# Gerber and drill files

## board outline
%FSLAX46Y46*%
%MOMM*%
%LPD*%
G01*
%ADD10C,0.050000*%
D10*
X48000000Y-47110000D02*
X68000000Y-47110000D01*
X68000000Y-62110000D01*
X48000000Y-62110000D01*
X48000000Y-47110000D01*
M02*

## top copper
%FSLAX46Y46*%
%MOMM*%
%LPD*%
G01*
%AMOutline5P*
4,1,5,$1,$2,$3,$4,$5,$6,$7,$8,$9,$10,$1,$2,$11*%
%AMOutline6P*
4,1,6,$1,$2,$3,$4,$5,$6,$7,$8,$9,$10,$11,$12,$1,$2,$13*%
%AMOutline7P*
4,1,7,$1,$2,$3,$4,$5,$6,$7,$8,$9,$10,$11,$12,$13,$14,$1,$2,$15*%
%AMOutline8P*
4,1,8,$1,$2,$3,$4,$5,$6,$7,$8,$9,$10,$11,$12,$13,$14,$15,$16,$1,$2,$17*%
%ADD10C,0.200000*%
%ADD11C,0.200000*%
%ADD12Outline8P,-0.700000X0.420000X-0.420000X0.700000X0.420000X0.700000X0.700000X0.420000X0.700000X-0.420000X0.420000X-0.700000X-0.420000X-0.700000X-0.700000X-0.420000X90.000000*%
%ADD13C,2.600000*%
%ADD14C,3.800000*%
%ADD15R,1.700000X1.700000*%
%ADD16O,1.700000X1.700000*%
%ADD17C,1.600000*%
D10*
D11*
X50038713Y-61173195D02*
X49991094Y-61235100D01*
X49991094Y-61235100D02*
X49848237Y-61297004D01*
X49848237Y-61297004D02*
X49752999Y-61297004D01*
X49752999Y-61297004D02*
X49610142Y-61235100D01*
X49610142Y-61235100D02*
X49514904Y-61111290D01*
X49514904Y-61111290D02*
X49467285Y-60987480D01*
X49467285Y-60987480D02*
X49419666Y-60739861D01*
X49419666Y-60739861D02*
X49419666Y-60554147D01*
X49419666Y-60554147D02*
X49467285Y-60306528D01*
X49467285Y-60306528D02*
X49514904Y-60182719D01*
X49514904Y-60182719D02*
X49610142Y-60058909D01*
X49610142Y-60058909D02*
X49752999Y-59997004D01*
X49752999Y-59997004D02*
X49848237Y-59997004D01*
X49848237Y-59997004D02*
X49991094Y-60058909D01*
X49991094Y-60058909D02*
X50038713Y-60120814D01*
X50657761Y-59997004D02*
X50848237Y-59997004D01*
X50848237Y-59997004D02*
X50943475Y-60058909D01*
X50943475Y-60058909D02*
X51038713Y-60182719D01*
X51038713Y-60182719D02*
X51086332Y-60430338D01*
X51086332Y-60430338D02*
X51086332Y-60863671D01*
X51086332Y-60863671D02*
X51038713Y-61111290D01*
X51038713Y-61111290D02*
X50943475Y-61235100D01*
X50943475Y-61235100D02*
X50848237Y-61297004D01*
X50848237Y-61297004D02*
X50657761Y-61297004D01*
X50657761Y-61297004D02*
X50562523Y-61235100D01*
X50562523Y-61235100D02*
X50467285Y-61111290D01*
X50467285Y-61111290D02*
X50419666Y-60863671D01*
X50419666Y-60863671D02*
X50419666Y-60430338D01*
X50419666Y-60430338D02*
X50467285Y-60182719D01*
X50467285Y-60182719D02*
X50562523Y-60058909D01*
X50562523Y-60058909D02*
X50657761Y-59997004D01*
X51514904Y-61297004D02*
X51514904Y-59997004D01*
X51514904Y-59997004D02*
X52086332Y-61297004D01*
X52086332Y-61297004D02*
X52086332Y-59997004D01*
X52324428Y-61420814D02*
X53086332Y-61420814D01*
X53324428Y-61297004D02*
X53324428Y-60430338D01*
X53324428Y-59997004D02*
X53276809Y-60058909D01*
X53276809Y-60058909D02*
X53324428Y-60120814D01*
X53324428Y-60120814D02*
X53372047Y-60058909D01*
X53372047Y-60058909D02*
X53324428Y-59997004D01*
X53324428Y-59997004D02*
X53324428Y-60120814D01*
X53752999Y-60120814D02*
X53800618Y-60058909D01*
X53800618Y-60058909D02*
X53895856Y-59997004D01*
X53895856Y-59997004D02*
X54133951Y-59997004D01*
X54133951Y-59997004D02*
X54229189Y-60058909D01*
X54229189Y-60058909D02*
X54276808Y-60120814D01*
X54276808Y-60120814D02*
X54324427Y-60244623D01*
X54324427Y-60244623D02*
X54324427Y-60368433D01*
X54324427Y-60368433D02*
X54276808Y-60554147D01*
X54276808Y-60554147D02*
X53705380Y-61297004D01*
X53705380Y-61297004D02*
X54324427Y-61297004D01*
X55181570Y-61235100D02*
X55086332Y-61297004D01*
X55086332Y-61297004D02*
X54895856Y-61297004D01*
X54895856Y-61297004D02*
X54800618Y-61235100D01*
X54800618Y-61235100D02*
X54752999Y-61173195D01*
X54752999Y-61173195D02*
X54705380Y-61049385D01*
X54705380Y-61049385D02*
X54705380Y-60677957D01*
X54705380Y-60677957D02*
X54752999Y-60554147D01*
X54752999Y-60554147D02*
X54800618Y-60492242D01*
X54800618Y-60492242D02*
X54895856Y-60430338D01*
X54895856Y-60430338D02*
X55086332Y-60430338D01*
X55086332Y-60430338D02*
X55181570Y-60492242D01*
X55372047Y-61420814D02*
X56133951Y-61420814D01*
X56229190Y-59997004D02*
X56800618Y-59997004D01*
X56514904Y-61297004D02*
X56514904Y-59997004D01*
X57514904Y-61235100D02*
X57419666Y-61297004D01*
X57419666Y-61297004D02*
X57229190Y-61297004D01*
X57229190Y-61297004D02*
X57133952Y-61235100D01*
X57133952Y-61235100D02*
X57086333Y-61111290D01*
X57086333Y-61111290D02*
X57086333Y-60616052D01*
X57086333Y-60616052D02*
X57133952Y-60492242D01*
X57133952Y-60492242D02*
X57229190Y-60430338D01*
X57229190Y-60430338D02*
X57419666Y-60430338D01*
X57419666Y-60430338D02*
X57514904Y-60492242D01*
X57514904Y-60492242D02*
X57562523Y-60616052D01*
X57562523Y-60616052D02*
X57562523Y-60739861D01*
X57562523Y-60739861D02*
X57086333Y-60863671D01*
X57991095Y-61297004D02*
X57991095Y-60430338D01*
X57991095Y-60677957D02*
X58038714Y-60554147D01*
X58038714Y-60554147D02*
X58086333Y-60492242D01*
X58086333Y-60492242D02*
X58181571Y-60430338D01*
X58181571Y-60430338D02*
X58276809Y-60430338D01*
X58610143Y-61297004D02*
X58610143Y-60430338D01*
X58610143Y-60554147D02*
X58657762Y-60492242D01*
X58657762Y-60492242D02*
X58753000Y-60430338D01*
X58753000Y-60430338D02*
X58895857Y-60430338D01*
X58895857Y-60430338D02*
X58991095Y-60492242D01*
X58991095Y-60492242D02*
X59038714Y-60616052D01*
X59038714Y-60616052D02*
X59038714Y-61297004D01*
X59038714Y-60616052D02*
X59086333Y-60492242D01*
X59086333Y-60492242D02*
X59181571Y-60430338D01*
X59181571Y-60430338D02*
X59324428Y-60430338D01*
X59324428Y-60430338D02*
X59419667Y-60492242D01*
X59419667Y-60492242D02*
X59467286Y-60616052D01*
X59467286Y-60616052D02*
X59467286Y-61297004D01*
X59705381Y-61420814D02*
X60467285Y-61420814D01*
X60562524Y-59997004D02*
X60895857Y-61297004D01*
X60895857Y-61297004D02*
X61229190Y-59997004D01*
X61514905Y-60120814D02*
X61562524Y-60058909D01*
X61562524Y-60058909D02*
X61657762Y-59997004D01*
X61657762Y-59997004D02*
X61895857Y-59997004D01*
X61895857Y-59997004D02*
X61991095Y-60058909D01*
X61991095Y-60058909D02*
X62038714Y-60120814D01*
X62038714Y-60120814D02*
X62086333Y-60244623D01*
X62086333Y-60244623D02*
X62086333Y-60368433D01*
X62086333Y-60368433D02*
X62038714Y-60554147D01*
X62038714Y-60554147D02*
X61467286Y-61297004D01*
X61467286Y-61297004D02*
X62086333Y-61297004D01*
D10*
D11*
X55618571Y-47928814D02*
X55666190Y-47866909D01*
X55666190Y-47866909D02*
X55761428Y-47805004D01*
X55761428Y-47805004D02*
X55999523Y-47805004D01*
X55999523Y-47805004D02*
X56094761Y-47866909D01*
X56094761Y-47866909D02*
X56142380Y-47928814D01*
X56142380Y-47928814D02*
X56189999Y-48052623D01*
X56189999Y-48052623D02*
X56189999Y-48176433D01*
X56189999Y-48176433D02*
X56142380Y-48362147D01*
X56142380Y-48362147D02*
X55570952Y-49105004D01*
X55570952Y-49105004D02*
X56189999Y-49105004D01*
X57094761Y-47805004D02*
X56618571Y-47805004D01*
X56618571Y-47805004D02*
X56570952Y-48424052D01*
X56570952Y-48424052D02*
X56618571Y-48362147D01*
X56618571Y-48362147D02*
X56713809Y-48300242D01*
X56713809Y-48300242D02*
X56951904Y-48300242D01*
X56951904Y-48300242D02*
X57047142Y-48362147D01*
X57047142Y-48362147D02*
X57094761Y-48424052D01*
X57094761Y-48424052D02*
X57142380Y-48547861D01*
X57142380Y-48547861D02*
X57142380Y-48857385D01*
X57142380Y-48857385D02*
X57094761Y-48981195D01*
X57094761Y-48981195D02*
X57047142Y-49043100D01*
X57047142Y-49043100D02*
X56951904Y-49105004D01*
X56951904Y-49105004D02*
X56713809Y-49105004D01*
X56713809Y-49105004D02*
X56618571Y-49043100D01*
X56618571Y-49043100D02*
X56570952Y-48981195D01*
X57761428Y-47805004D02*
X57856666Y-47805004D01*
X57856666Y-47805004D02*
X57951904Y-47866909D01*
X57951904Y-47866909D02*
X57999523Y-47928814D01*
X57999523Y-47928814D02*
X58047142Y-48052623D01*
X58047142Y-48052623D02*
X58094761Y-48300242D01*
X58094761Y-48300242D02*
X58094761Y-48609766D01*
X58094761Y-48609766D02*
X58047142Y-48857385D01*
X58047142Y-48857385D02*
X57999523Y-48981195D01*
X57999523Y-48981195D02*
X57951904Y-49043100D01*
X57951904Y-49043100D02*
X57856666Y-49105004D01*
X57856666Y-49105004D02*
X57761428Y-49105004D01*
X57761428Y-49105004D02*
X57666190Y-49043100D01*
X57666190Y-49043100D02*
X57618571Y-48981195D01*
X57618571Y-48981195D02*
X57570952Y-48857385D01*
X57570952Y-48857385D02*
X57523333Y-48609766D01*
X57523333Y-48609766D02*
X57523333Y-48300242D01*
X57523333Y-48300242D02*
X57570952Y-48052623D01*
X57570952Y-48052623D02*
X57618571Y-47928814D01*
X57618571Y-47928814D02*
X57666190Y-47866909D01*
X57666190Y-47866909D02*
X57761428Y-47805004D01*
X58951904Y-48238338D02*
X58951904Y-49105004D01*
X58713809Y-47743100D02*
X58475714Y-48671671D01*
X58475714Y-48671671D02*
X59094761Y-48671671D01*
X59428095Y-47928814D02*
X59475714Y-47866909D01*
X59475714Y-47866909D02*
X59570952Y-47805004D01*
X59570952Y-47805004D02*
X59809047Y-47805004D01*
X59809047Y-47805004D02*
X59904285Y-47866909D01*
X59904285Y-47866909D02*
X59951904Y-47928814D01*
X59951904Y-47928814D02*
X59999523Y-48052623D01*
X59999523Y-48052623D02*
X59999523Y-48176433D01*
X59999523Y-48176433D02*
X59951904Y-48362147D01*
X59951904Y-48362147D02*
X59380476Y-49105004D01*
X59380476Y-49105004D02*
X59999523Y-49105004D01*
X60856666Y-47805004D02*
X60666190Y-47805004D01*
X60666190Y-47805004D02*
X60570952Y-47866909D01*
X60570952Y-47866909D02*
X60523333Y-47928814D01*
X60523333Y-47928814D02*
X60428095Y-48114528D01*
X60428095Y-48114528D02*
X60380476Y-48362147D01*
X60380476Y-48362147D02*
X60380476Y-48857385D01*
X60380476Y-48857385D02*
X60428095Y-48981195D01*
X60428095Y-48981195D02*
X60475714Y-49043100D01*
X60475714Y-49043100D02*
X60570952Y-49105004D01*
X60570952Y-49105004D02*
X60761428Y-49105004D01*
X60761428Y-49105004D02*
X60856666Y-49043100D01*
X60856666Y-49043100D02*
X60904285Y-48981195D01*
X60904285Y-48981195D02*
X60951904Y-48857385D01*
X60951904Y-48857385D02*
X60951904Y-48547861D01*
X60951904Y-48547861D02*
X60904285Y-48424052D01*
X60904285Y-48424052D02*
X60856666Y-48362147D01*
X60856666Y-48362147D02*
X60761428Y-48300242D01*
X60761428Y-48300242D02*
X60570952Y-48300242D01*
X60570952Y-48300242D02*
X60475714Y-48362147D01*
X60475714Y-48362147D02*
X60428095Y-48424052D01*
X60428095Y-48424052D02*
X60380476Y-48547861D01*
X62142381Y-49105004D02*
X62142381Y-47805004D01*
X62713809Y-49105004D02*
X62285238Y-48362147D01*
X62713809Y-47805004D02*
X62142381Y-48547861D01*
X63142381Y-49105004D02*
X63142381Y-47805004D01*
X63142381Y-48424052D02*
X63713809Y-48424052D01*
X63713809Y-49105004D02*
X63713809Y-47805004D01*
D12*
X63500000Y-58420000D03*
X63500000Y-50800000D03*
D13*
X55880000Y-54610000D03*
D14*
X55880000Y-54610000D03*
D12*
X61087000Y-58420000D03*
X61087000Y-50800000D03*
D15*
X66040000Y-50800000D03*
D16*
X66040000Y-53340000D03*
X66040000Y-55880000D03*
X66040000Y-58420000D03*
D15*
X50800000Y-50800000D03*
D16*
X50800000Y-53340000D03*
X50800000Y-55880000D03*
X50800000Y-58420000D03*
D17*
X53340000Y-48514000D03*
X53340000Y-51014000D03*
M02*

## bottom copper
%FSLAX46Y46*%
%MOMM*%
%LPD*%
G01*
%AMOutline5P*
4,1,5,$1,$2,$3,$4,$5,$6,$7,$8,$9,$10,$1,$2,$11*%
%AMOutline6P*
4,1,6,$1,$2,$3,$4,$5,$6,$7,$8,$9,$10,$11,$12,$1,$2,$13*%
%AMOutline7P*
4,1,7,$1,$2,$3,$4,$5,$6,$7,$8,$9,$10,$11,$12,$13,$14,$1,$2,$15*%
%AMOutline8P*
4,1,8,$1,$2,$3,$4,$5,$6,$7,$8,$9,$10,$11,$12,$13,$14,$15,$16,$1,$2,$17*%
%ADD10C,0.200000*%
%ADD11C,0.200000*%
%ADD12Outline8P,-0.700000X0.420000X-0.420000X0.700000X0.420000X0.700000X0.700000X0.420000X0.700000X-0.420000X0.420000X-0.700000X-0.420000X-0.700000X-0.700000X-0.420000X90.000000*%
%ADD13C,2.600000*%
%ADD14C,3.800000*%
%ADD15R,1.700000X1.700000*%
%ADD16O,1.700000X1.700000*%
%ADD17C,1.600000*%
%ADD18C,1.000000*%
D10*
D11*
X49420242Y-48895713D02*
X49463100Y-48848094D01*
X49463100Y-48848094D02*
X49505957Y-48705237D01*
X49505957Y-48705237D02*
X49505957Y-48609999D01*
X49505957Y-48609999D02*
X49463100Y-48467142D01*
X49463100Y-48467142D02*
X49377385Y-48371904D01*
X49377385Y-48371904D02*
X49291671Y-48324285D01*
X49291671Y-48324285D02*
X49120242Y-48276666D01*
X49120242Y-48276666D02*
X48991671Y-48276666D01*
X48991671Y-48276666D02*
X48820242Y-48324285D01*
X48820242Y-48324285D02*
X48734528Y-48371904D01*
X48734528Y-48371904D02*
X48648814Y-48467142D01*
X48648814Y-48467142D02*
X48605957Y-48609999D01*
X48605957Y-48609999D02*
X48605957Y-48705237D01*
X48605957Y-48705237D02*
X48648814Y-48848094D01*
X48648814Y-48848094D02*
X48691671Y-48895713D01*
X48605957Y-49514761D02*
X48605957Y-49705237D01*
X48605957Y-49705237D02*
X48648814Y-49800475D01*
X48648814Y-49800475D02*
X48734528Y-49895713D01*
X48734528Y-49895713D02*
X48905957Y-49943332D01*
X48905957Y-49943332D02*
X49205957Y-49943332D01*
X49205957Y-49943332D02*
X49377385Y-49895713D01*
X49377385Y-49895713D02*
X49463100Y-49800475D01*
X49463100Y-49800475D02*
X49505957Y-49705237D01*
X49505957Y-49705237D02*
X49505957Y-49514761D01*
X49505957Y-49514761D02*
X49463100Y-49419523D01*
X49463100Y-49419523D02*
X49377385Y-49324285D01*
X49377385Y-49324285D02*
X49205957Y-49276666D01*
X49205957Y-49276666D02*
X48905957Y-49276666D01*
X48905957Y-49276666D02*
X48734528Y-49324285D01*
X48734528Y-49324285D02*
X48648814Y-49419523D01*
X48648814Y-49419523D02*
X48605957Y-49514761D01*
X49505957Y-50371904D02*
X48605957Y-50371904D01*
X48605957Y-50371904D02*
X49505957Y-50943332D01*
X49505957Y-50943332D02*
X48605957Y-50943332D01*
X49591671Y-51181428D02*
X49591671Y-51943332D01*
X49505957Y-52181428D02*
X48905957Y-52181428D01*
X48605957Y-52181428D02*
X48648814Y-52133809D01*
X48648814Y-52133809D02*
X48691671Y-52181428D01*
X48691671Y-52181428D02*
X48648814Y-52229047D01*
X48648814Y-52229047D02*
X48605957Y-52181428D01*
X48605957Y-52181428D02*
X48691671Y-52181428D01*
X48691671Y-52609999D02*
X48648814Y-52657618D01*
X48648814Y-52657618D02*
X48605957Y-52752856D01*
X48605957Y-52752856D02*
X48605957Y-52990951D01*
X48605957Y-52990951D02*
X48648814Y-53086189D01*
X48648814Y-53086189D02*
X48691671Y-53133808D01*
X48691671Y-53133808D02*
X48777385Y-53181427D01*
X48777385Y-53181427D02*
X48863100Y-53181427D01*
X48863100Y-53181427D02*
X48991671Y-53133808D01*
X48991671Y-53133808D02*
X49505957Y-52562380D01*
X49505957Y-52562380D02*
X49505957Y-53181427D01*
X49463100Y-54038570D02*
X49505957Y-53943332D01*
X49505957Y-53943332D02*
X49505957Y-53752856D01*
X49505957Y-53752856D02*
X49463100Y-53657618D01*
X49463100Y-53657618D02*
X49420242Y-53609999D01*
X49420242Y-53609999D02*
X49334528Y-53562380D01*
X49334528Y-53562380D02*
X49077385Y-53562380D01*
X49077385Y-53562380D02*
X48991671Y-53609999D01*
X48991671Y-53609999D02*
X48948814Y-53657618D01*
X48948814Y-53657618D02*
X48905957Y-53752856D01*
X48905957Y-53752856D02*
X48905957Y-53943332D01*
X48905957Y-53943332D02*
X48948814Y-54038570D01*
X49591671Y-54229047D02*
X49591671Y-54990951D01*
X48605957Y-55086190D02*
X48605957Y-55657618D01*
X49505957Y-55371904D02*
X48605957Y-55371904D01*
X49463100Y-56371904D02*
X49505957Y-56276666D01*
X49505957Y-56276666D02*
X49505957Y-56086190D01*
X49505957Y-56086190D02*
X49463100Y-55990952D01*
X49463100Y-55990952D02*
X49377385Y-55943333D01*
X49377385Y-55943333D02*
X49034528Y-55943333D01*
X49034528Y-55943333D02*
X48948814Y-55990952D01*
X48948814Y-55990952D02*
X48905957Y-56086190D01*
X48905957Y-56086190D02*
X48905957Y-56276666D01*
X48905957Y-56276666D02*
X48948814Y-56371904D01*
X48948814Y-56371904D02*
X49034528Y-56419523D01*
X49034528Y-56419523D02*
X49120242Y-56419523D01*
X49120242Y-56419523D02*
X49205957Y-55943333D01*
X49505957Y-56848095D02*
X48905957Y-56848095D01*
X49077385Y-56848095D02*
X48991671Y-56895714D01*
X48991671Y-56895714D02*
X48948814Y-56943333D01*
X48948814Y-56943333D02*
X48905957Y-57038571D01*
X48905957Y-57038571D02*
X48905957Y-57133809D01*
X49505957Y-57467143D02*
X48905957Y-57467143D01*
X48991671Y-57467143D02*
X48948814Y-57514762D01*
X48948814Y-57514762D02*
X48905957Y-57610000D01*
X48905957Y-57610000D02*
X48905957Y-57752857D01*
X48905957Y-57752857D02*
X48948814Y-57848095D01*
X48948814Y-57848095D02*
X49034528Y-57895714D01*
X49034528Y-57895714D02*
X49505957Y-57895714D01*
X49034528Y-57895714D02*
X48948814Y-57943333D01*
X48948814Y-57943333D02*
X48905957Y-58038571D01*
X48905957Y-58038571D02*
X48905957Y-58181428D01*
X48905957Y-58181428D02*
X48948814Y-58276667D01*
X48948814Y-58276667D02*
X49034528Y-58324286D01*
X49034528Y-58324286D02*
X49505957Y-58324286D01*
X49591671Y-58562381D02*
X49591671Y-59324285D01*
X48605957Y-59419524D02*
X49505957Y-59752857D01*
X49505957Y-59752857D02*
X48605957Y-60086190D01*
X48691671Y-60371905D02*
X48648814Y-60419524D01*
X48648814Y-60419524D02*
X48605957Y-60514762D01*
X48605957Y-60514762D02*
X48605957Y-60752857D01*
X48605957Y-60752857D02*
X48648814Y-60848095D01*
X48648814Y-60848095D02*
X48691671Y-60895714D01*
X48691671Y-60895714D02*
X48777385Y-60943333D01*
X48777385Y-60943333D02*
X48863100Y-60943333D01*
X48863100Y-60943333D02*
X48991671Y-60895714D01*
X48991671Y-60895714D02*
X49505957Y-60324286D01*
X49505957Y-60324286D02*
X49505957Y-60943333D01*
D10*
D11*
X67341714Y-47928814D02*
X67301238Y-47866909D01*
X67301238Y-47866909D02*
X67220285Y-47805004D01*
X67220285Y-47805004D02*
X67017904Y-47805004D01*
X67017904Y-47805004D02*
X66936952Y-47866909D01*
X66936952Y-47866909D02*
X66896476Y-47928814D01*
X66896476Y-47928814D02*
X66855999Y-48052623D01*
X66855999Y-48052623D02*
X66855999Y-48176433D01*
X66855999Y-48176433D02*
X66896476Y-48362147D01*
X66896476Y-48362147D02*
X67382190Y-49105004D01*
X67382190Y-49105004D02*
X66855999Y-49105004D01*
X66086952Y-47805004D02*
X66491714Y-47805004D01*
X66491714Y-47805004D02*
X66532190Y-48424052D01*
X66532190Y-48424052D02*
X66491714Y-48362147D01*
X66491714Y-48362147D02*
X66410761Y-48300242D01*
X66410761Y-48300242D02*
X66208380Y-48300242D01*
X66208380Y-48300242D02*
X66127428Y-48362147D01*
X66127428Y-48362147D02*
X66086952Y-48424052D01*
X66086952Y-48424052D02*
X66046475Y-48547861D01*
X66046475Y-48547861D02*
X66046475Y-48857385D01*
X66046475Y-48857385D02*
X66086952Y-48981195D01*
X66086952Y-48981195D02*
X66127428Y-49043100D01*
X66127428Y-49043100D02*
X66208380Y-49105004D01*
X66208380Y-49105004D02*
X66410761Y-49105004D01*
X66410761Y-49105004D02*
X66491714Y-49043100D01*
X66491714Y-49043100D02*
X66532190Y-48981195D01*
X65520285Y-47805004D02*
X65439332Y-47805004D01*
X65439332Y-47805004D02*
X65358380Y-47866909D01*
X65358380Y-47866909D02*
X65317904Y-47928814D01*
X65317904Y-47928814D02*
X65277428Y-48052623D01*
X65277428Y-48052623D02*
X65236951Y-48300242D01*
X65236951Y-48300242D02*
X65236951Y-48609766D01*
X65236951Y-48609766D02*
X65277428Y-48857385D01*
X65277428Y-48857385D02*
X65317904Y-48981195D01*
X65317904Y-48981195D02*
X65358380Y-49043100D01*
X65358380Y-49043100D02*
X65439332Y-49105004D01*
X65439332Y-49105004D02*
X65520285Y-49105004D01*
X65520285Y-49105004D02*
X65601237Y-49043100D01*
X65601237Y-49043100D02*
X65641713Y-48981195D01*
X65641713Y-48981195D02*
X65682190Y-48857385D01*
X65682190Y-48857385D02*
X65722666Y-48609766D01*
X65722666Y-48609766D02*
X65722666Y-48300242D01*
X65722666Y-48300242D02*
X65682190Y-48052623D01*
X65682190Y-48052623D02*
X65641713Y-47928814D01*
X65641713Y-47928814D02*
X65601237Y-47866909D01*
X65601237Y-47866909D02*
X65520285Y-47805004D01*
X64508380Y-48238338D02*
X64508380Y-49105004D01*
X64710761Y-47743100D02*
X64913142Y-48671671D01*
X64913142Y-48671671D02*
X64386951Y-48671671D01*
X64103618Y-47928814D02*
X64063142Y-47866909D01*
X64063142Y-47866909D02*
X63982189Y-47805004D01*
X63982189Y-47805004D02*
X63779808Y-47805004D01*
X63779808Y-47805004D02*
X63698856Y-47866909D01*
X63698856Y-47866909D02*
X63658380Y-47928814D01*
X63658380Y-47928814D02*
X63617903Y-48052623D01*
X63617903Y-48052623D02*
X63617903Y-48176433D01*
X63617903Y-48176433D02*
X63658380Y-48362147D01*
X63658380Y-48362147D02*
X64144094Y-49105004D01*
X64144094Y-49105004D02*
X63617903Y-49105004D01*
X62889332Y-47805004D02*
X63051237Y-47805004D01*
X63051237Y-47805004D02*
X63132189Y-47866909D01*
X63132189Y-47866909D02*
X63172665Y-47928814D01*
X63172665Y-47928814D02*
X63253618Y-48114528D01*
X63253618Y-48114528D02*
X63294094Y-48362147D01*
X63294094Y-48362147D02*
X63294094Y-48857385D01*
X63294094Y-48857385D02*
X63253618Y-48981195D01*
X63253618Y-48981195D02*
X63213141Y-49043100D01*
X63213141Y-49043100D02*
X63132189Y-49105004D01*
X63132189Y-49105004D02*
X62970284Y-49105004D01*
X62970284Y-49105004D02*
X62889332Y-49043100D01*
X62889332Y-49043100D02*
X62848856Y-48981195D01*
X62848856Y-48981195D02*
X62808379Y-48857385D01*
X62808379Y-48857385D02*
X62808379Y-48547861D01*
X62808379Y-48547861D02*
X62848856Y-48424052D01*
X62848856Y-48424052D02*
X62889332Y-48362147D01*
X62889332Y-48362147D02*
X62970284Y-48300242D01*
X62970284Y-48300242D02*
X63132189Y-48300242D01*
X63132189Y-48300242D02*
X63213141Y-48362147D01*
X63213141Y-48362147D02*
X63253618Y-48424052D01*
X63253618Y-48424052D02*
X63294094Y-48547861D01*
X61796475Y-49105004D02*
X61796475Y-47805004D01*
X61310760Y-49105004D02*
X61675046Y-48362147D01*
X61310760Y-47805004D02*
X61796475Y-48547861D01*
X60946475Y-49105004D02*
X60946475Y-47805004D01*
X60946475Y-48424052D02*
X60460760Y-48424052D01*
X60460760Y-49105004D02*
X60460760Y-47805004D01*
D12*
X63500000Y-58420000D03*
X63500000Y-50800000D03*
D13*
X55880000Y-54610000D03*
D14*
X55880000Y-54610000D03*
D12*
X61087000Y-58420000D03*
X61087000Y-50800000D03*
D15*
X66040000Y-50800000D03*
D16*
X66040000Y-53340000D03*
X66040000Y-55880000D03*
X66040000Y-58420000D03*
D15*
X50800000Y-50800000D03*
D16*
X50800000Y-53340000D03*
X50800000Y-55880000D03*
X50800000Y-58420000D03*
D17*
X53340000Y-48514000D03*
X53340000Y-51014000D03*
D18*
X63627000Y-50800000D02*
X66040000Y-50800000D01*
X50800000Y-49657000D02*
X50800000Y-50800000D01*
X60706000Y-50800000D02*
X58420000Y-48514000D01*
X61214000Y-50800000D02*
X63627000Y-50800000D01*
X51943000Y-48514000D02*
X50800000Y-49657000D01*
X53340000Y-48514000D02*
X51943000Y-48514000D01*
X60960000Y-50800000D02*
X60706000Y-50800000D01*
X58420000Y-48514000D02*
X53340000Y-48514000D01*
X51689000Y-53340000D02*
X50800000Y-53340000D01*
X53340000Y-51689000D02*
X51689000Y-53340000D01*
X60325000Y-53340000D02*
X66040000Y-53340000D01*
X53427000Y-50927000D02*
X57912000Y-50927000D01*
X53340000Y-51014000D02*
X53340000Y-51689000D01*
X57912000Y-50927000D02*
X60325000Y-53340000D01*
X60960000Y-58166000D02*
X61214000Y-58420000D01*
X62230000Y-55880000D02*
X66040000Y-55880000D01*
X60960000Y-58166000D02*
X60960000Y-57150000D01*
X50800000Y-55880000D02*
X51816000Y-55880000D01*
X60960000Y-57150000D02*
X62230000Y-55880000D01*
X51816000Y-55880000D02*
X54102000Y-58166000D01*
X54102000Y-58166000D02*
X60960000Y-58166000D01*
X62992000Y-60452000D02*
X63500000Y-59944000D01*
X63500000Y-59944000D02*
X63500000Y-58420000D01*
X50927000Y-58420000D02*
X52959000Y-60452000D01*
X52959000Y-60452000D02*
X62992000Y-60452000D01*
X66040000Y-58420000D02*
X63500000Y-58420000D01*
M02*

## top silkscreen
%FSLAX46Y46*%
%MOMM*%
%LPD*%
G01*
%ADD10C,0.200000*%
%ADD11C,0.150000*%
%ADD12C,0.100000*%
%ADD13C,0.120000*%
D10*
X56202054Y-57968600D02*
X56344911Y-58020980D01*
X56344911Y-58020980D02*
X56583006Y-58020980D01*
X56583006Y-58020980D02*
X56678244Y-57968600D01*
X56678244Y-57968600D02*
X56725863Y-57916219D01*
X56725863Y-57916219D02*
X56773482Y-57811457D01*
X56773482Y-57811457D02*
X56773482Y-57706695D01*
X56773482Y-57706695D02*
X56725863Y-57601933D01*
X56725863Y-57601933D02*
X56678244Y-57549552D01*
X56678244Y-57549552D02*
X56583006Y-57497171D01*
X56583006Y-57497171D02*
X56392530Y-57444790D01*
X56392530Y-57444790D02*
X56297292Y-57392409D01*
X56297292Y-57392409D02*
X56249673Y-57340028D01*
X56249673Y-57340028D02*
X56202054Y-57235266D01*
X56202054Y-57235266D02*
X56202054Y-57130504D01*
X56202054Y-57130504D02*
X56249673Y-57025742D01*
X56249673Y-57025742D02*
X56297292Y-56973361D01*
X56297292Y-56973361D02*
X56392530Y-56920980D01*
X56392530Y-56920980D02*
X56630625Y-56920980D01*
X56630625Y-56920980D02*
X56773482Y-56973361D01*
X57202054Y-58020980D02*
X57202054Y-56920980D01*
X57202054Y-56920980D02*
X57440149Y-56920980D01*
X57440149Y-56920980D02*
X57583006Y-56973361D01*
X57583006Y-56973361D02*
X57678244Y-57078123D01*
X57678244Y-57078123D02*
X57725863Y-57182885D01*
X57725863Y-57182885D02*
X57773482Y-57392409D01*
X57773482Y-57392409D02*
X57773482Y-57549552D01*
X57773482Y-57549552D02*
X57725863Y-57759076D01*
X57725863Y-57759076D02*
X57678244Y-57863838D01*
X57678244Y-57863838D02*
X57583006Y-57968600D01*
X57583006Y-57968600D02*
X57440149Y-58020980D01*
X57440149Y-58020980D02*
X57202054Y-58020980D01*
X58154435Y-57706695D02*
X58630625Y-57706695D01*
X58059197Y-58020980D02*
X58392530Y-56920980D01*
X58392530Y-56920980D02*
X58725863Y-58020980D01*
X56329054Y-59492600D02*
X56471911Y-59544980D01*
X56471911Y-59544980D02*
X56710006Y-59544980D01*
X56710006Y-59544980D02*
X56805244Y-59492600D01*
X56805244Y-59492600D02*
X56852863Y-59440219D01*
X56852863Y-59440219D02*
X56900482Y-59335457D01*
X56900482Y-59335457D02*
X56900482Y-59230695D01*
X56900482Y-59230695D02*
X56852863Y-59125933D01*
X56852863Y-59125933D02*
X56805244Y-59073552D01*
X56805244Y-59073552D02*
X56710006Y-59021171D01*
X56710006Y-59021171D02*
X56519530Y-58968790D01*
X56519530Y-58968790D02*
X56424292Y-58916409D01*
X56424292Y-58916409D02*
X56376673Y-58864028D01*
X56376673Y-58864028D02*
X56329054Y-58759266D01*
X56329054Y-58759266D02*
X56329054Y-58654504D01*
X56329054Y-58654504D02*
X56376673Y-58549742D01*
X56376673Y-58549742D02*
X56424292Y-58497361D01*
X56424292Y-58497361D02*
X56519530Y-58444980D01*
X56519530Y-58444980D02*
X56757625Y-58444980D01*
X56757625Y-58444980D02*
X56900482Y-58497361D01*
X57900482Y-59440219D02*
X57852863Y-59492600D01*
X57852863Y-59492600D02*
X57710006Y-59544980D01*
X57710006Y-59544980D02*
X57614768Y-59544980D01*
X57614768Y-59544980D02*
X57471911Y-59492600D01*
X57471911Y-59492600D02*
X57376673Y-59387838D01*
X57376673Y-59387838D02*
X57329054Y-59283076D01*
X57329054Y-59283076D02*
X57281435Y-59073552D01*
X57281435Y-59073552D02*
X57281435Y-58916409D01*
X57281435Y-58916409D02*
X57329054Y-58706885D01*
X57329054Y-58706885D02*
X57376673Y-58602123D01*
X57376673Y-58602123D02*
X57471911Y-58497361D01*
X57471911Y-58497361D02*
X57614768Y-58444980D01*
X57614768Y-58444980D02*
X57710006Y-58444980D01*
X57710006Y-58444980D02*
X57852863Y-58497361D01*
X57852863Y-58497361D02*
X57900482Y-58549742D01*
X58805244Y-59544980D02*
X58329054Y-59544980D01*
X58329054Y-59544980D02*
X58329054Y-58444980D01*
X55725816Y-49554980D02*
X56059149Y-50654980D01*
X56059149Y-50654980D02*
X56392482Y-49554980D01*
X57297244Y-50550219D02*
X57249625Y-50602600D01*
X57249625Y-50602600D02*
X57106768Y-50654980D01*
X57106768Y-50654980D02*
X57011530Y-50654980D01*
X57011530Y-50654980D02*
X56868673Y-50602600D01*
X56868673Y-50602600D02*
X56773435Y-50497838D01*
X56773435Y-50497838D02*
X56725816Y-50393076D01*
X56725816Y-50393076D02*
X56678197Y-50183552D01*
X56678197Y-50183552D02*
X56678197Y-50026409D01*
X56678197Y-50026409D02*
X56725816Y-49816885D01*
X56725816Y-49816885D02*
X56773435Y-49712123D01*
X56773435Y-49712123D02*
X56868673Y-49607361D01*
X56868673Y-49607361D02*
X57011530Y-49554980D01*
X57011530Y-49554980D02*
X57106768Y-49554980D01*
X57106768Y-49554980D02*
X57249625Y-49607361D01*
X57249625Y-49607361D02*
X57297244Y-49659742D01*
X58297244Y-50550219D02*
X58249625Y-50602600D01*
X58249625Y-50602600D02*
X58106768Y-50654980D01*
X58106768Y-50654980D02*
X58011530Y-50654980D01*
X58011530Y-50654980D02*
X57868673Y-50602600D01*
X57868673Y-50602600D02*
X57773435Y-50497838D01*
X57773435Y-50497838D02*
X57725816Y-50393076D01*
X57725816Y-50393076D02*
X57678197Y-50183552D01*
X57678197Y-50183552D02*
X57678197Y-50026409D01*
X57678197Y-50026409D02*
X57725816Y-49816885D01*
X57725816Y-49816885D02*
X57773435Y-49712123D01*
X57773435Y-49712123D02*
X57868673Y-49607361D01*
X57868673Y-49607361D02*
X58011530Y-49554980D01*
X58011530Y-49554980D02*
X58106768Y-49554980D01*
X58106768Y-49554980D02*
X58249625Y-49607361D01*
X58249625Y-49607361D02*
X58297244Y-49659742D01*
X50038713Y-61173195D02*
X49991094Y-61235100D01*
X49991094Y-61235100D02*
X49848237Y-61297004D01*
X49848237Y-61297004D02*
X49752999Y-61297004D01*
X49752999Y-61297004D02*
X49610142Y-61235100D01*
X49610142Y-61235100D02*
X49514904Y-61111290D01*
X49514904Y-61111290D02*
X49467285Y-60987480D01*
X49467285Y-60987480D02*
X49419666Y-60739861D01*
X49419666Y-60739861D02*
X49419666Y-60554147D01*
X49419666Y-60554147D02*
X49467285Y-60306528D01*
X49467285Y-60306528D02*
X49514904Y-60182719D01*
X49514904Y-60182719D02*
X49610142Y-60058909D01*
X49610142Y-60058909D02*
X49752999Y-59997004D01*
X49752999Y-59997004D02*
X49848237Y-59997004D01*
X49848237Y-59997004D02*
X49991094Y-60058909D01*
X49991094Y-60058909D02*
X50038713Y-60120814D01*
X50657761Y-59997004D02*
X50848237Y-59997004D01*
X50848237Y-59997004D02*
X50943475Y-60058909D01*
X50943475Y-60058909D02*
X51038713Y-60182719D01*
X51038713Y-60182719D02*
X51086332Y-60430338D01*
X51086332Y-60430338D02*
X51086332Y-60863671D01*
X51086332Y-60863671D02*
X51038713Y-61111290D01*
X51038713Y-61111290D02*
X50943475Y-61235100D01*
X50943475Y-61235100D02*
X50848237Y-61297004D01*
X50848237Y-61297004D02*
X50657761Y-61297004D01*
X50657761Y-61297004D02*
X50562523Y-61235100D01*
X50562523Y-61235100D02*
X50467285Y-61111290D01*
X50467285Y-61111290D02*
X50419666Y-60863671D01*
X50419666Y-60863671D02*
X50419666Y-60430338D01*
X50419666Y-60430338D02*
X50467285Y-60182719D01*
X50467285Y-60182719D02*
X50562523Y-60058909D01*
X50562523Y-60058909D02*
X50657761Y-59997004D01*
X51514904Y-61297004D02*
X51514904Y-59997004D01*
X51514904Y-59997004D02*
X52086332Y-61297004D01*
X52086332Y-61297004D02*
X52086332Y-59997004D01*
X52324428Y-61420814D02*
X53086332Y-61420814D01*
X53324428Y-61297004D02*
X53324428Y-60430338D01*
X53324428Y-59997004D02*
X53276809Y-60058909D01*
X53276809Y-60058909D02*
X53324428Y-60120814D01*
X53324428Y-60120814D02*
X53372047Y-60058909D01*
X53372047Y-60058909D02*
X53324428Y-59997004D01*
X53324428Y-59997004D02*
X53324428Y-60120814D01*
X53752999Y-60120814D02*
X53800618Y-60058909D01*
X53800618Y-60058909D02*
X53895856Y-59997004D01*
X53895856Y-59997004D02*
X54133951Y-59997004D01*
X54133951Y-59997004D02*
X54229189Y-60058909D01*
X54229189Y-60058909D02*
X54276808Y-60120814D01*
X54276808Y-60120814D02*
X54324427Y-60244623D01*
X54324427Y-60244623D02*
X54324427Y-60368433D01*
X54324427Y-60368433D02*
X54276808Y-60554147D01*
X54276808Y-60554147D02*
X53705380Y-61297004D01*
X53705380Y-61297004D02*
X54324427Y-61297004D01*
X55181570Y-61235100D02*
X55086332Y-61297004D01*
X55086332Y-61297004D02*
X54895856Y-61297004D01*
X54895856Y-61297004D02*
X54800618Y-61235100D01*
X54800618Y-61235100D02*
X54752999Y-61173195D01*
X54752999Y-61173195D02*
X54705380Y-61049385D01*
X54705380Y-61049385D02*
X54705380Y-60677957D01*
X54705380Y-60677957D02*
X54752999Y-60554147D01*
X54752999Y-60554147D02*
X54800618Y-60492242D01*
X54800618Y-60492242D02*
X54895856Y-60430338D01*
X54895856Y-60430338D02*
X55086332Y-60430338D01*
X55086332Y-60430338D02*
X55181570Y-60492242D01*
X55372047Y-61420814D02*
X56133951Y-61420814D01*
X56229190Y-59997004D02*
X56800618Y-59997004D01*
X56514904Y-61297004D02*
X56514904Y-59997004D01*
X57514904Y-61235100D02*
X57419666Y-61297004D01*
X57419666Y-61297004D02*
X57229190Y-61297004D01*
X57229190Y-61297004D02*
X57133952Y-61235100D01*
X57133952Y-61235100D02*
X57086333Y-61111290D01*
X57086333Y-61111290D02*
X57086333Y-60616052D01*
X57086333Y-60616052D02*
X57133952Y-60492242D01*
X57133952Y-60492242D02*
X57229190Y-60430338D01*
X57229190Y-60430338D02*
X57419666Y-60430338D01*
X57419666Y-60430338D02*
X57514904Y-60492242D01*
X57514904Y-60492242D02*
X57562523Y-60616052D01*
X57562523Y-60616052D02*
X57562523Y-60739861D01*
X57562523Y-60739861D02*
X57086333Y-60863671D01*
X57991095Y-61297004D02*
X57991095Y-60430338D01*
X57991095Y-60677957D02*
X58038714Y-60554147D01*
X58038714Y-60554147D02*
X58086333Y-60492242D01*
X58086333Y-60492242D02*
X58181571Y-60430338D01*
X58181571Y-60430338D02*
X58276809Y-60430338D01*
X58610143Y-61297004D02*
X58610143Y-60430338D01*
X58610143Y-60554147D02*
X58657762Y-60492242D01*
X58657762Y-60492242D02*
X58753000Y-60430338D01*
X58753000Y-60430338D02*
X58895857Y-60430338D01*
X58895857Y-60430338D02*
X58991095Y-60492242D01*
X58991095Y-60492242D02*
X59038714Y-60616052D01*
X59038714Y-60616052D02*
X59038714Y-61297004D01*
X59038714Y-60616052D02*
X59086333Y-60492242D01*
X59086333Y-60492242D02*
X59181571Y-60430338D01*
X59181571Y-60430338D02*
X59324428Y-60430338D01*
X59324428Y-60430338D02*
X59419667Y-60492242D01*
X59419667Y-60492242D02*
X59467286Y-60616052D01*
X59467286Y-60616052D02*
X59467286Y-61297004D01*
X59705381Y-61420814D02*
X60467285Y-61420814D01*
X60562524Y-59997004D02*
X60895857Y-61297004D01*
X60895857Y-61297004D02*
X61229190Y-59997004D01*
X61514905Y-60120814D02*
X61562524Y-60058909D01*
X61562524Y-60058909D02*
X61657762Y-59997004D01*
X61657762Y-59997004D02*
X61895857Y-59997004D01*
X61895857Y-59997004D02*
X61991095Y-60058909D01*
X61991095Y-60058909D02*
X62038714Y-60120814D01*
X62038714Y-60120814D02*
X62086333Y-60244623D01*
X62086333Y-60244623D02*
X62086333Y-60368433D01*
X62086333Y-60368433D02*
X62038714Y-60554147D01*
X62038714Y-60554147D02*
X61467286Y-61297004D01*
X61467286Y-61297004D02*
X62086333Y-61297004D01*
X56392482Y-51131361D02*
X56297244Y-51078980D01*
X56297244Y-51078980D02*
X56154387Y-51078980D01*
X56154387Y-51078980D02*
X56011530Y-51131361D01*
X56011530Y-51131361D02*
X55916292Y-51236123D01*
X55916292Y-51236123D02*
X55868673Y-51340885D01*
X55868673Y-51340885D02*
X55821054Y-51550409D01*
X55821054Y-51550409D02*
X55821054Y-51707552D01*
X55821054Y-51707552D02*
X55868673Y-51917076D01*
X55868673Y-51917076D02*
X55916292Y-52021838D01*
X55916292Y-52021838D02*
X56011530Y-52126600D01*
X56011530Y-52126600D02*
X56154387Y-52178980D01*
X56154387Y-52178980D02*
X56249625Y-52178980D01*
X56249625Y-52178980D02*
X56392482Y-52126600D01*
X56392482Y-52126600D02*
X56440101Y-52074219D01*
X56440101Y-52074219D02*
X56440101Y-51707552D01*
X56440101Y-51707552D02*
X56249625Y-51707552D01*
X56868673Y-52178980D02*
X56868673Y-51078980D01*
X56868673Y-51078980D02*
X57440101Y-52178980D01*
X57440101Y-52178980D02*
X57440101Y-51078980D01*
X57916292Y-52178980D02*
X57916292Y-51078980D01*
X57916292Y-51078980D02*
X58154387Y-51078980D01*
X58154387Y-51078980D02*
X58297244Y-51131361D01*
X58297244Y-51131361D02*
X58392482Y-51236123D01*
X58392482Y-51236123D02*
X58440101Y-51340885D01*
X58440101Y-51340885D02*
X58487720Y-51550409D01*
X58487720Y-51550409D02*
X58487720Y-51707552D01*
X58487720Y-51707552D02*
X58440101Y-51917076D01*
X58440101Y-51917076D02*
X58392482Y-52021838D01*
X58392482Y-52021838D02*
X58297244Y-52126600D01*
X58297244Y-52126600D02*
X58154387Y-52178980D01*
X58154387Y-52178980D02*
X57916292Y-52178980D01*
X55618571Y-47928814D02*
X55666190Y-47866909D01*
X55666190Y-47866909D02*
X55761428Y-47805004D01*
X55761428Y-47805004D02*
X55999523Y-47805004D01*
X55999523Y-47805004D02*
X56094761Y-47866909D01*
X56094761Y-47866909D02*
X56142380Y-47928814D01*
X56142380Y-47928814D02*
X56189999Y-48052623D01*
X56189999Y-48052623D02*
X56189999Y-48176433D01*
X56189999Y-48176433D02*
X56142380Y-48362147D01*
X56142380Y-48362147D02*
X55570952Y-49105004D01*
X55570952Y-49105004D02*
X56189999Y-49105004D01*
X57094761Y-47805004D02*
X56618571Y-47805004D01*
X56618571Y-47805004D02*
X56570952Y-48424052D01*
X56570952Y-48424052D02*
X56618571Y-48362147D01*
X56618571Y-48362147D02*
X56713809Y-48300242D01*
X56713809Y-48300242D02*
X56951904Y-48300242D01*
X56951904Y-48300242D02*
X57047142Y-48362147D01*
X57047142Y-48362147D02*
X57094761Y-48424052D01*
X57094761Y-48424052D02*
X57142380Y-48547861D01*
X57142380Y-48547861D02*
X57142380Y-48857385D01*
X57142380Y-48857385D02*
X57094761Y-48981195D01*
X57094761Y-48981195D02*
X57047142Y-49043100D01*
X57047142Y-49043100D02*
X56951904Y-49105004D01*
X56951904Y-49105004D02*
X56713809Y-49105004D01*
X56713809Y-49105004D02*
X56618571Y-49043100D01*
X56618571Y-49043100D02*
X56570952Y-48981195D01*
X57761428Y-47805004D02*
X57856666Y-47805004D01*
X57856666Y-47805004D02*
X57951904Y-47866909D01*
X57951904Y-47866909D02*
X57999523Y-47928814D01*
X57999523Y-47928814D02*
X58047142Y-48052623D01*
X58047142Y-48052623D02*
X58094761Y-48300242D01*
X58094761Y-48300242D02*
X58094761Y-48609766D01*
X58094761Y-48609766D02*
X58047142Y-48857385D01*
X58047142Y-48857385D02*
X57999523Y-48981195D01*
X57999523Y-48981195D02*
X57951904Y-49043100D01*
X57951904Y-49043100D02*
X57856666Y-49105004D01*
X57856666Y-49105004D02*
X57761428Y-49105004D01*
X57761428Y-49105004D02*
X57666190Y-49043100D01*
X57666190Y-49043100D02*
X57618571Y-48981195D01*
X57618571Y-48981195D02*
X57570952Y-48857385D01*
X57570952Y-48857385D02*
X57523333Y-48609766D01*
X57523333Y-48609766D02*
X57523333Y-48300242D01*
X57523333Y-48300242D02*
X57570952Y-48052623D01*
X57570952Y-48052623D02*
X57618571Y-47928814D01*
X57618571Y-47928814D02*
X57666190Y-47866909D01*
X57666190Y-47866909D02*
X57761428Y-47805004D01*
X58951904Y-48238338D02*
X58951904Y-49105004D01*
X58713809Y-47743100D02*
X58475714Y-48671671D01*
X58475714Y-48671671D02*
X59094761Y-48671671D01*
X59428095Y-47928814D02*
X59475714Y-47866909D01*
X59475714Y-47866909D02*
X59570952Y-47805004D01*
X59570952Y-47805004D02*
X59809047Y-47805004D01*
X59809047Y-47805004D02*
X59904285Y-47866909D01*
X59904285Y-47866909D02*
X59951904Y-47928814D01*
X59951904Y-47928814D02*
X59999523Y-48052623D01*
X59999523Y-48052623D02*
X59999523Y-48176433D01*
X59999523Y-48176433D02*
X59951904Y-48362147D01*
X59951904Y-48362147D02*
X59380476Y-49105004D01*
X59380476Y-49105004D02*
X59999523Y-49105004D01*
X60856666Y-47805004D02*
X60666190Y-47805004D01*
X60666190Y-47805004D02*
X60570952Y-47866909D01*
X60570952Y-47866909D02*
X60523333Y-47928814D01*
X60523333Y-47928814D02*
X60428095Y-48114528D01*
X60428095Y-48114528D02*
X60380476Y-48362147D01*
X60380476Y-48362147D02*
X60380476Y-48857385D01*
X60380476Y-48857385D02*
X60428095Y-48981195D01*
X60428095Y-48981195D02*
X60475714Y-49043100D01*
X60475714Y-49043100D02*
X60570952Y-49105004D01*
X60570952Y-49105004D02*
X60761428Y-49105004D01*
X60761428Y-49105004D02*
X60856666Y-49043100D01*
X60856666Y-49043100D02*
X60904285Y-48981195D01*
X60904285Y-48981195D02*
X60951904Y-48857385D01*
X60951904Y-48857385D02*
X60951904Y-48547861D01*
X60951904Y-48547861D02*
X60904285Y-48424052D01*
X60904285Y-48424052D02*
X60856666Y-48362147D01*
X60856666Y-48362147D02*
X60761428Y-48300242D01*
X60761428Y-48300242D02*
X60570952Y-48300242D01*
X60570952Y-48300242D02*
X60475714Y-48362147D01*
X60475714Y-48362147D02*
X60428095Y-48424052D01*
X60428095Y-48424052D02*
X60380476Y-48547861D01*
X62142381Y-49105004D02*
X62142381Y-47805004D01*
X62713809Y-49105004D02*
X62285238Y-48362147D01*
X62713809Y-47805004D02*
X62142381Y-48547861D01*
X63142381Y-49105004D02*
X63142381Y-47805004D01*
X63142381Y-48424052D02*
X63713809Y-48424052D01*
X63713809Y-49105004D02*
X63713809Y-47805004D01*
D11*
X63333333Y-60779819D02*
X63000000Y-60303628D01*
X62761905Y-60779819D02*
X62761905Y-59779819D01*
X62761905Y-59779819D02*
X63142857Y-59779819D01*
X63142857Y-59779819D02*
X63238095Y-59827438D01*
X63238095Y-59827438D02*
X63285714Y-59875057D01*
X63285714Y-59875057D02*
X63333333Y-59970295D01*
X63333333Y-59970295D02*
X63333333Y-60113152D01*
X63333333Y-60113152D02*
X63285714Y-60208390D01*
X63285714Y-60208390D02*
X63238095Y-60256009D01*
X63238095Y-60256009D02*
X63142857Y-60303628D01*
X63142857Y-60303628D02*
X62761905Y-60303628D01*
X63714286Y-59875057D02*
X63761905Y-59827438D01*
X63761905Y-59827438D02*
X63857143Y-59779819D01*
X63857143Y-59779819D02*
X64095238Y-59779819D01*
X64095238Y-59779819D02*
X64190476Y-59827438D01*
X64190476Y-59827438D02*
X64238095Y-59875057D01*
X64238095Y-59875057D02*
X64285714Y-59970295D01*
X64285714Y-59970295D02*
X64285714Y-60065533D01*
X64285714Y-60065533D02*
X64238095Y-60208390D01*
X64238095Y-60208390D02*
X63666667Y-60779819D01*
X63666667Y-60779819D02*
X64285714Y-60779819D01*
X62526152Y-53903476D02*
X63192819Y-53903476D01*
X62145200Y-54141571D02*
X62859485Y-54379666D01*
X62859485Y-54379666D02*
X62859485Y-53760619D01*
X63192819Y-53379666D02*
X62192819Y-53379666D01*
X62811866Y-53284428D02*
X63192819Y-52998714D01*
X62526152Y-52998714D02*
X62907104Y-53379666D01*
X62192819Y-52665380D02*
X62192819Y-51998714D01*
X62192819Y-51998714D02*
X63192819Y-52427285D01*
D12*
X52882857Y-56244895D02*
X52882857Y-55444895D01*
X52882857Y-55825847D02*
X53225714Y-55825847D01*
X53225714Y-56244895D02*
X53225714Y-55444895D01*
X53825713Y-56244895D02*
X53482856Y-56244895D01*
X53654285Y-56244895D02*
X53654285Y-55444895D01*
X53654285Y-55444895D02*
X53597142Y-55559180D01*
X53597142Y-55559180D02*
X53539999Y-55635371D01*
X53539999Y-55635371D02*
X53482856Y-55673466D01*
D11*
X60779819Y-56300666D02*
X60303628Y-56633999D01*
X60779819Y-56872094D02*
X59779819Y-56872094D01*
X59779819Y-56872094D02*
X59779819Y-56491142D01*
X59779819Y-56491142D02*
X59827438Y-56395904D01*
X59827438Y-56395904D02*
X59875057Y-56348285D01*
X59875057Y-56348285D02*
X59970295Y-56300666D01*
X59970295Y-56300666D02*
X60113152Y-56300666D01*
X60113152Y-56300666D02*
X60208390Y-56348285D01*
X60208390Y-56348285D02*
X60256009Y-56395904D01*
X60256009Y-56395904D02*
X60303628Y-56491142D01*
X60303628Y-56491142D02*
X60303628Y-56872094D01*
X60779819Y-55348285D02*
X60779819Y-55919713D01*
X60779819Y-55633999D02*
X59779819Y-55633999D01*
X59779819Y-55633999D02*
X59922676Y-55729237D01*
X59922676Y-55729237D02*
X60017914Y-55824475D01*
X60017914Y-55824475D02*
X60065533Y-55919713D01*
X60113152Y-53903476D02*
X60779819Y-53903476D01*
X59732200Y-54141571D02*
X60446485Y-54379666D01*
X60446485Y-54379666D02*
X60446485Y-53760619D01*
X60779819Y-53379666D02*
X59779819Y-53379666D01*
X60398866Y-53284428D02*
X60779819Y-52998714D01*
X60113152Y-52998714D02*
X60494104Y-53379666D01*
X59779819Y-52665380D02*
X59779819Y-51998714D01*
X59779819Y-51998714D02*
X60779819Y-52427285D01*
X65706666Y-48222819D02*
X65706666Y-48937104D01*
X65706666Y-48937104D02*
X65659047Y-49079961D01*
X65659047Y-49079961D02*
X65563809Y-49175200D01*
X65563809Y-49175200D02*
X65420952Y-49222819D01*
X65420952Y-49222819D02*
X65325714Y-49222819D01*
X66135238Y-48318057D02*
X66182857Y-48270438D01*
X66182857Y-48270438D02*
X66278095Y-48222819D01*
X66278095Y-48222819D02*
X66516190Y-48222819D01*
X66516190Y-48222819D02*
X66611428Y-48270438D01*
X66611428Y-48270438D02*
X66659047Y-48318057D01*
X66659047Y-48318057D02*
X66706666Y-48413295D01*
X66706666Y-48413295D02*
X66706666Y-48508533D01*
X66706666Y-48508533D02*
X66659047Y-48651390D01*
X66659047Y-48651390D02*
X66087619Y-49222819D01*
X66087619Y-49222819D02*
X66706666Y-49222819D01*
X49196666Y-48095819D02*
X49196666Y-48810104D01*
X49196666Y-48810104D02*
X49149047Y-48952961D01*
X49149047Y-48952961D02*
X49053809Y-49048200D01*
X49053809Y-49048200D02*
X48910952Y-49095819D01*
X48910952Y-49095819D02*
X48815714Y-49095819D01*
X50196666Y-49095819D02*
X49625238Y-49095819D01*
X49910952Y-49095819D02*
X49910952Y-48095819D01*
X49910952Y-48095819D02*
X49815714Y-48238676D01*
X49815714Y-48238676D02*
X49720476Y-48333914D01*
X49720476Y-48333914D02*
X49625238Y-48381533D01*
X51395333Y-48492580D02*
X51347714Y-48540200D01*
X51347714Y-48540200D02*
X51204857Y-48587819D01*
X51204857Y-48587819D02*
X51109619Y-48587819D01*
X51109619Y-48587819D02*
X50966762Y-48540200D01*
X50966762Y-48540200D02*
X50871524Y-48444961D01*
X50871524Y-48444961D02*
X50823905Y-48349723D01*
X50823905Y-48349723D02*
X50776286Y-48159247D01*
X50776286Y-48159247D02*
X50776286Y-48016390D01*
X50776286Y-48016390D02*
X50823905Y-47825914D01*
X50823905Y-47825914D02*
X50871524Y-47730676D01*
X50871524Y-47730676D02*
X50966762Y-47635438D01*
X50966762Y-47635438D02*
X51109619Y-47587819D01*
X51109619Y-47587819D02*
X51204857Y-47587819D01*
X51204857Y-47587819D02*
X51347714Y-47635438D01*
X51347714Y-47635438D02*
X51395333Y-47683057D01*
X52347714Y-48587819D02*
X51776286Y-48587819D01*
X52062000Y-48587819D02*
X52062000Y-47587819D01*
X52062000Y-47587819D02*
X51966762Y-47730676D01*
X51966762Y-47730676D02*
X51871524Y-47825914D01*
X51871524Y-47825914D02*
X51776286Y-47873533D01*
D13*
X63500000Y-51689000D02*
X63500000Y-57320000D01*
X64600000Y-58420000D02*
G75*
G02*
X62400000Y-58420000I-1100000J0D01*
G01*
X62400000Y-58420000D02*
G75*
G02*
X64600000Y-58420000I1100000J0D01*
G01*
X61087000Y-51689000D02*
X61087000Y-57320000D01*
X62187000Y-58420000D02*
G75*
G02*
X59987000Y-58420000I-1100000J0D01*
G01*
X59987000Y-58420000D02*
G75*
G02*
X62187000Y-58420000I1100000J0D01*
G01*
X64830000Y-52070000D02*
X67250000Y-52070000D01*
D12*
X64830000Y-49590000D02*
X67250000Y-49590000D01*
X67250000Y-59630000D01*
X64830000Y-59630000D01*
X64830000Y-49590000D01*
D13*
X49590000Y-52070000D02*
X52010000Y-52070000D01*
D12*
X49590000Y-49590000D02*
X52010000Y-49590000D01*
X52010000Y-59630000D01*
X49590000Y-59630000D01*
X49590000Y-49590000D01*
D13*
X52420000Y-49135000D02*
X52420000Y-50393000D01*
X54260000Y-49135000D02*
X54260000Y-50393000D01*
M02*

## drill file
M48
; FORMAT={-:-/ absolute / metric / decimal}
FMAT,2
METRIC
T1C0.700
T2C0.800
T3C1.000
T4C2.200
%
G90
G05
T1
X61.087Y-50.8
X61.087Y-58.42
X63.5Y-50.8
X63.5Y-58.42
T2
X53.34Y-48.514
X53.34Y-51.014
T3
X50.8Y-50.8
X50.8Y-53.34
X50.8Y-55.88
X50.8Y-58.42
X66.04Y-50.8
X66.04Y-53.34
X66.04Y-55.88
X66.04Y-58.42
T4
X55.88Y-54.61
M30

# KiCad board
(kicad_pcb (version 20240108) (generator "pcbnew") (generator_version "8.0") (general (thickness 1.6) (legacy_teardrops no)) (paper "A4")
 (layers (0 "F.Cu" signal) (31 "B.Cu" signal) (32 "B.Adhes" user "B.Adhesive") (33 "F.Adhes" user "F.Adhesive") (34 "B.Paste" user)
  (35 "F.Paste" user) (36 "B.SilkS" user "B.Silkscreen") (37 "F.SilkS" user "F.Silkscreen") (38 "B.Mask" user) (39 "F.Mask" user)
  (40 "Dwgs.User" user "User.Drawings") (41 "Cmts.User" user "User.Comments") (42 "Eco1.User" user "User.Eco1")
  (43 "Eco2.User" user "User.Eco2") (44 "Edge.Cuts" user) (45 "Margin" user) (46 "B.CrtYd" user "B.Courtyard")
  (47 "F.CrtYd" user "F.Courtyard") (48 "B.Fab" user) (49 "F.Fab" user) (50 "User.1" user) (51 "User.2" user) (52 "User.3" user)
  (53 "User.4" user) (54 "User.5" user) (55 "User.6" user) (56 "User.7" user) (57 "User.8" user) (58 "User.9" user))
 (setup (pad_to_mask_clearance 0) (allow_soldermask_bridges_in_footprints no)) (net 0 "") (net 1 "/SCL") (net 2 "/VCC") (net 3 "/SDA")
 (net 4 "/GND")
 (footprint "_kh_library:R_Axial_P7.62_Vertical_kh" (layer "F.Cu") (at 63.5 58.42 90)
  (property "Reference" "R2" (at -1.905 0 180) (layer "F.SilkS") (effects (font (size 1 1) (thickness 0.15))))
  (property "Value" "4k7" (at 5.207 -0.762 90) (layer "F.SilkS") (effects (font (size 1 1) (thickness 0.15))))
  (fp_line (start 6.731 0) (end 1.1 0) (stroke (width 0.12) (type solid)) (layer "F.SilkS"))
  (fp_circle (center 0 0) (end 1.1 0) (stroke (width 0.12) (type solid)) (fill none) (layer "F.SilkS"))
  (pad "1" thru_hole roundrect (at 0 0 90) (size 1.4 1.4) (drill 0.7) (layers "*.Cu" "*.Mask") (remove_unused_layers no)
   (roundrect_rratio 0) (chamfer_ratio 0.2) (chamfer top_left top_right bottom_left bottom_right) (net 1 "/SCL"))
  (pad "2" thru_hole roundrect (at 7.62 0 90) (size 1.4 1.4) (drill 0.7) (layers "*.Cu" "*.Mask") (remove_unused_layers no)
   (roundrect_rratio 0) (chamfer_ratio 0.2) (chamfer top_left top_right bottom_left bottom_right) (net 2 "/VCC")))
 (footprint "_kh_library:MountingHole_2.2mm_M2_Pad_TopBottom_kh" (layer "F.Cu") (at 55.88 54.61)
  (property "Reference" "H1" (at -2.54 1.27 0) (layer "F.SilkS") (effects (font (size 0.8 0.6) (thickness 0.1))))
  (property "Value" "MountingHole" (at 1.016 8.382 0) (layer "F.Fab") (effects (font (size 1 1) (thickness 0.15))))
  (pad "1" thru_hole circle (at 0 0) (size 2.6 2.6) (drill 2.2) (layers "*.Cu" "*.Mask") (remove_unused_layers no))
  (pad "1" connect circle (at 0 0) (size 3.8 3.8) (layers "F.Cu" "F.Mask"))
  (pad "1" connect circle (at 0 0) (size 3.8 3.8) (layers "B.Cu" "B.Mask")))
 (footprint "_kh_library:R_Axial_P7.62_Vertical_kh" (layer "F.Cu") (at 61.087 58.42 90)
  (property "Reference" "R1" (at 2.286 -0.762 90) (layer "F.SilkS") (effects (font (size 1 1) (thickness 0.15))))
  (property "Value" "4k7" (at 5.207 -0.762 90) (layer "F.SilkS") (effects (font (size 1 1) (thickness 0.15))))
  (fp_line (start 6.731 0) (end 1.1 0) (stroke (width 0.12) (type solid)) (layer "F.SilkS"))
  (fp_circle (center 0 0) (end 1.1 0) (stroke (width 0.12) (type solid)) (fill none) (layer "F.SilkS"))
  (pad "1" thru_hole roundrect (at 0 0 90) (size 1.4 1.4) (drill 0.7) (layers "*.Cu" "*.Mask") (remove_unused_layers no)
   (roundrect_rratio 0) (chamfer_ratio 0.2) (chamfer top_left top_right bottom_left bottom_right) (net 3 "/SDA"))
  (pad "2" thru_hole roundrect (at 7.62 0 90) (size 1.4 1.4) (drill 0.7) (layers "*.Cu" "*.Mask") (remove_unused_layers no)
   (roundrect_rratio 0) (chamfer_ratio 0.2) (chamfer top_left top_right bottom_left bottom_right) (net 2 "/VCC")))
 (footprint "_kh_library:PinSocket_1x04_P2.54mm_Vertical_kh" (layer "F.Cu") (at 66.04 50.8)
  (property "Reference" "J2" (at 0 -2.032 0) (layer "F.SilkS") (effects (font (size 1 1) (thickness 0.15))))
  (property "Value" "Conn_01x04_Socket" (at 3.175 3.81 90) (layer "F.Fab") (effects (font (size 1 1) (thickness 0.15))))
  (fp_line (start -1.21 1.27) (end 1.21 1.27) (stroke (width 0.12) (type solid)) (layer "F.SilkS"))
  (fp_rect (start -1.21 -1.21) (end 1.21 8.83) (stroke (width 0.1) (type default)) (fill none) (layer "F.SilkS"))
  (pad "1" thru_hole rect (at 0 0) (size 1.7 1.7) (drill 1) (layers "*.Cu" "*.Mask") (remove_unused_layers no) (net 2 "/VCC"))
  (pad "2" thru_hole oval (at 0 2.54) (size 1.7 1.7) (drill 1) (layers "*.Cu" "*.Mask") (remove_unused_layers no) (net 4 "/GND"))
  (pad "3" thru_hole oval (at 0 5.08) (size 1.7 1.7) (drill 1) (layers "*.Cu" "*.Mask") (remove_unused_layers no) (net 3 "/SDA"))
  (pad "4" thru_hole oval (at 0 7.62) (size 1.7 1.7) (drill 1) (layers "*.Cu" "*.Mask") (remove_unused_layers no) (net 1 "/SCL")))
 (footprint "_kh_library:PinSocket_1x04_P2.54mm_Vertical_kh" (layer "F.Cu") (at 50.8 50.8)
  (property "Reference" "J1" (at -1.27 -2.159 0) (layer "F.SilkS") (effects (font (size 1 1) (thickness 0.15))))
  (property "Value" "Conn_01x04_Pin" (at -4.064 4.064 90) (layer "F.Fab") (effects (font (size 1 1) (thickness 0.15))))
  (fp_line (start -1.21 1.27) (end 1.21 1.27) (stroke (width 0.12) (type solid)) (layer "F.SilkS"))
  (fp_rect (start -1.21 -1.21) (end 1.21 8.83) (stroke (width 0.1) (type default)) (fill none) (layer "F.SilkS"))
  (pad "1" thru_hole rect (at 0 0) (size 1.7 1.7) (drill 1) (layers "*.Cu" "*.Mask") (remove_unused_layers no) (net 2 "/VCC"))
  (pad "2" thru_hole oval (at 0 2.54) (size 1.7 1.7) (drill 1) (layers "*.Cu" "*.Mask") (remove_unused_layers no) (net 4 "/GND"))
  (pad "3" thru_hole oval (at 0 5.08) (size 1.7 1.7) (drill 1) (layers "*.Cu" "*.Mask") (remove_unused_layers no) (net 3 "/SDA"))
  (pad "4" thru_hole oval (at 0 7.62) (size 1.7 1.7) (drill 1) (layers "*.Cu" "*.Mask") (remove_unused_layers no) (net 1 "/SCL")))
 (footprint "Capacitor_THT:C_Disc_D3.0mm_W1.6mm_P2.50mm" (layer "F.Cu") (at 53.34 48.514 -90)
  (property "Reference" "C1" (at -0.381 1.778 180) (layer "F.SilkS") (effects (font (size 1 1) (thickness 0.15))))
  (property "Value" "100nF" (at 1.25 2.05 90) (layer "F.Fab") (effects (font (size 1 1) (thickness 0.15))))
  (fp_line (start 0.621 0.92) (end 1.879 0.92) (stroke (width 0.12) (type solid)) (layer "F.SilkS"))
  (fp_line (start 0.621 -0.92) (end 1.879 -0.92) (stroke (width 0.12) (type solid)) (layer "F.SilkS"))
  (pad "1" thru_hole circle (at 0 0 270) (size 1.6 1.6) (drill 0.8) (layers "*.Cu" "*.Mask") (remove_unused_layers no) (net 2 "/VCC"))
  (pad "2" thru_hole circle (at 2.5 0 270) (size 1.6 1.6) (drill 0.8) (layers "*.Cu" "*.Mask") (remove_unused_layers no) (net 4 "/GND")))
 (gr_rect (start 48 47.11) (end 68 62.11) (stroke (width 0.05) (type default)) (fill none) (layer "Edge.Cuts"))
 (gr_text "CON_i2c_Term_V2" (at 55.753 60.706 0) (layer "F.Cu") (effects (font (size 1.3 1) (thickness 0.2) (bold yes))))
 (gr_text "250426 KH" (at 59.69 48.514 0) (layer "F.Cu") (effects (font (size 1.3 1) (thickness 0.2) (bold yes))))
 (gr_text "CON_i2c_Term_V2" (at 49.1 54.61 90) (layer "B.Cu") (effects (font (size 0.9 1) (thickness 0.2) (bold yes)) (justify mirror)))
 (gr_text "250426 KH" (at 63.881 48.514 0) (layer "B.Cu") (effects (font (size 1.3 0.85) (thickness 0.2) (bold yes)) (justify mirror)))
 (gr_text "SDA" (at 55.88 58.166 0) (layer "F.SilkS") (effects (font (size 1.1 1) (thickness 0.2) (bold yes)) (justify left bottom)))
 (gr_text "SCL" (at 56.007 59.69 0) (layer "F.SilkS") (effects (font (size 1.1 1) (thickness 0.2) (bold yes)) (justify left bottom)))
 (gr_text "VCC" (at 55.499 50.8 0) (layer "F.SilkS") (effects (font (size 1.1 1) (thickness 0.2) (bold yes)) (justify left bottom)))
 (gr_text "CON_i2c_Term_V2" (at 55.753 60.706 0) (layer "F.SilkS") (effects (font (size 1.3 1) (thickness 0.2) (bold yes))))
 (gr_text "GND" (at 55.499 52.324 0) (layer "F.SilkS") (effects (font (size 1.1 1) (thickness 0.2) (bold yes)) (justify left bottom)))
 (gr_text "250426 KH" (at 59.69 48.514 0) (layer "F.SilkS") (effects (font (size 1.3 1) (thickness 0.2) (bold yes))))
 (segment (start 63.627 50.8) (end 66.04 50.8) (width 1) (layer "B.Cu") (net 2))
 (segment (start 50.8 49.657) (end 50.8 50.8) (width 1) (layer "B.Cu") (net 2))
 (segment (start 60.706 50.8) (end 58.42 48.514) (width 1) (layer "B.Cu") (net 2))
 (segment (start 61.214 50.8) (end 63.627 50.8) (width 1) (layer "B.Cu") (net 2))
 (segment (start 51.943 48.514) (end 50.8 49.657) (width 1) (layer "B.Cu") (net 2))
 (segment (start 53.34 48.514) (end 51.943 48.514) (width 1) (layer "B.Cu") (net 2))
 (segment (start 60.96 50.8) (end 60.706 50.8) (width 1) (layer "B.Cu") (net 2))
 (segment (start 58.42 48.514) (end 53.34 48.514) (width 1) (layer "B.Cu") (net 2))
 (segment (start 51.689 53.34) (end 50.8 53.34) (width 1) (layer "B.Cu") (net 4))
 (segment (start 53.34 51.689) (end 51.689 53.34) (width 1) (layer "B.Cu") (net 4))
 (segment (start 60.325 53.34) (end 66.04 53.34) (width 1) (layer "B.Cu") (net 4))
 (segment (start 53.427 50.927) (end 57.912 50.927) (width 1) (layer "B.Cu") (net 4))
 (segment (start 53.34 51.014) (end 53.34 51.689) (width 1) (layer "B.Cu") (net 4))
 (segment (start 57.912 50.927) (end 60.325 53.34) (width 1) (layer "B.Cu") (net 4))
 (segment (start 60.96 58.166) (end 61.214 58.42) (width 1) (layer "B.Cu") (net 3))
 (segment (start 62.23 55.88) (end 66.04 55.88) (width 1) (layer "B.Cu") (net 3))
 (segment (start 60.96 58.166) (end 60.96 57.15) (width 1) (layer "B.Cu") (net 3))
 (segment (start 50.8 55.88) (end 51.816 55.88) (width 1) (layer "B.Cu") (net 3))
 (segment (start 60.96 57.15) (end 62.23 55.88) (width 1) (layer "B.Cu") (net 3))
 (segment (start 51.816 55.88) (end 54.102 58.166) (width 1) (layer "B.Cu") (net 3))
 (segment (start 54.102 58.166) (end 60.96 58.166) (width 1) (layer "B.Cu") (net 3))
 (segment (start 62.992 60.452) (end 63.5 59.944) (width 1) (layer "B.Cu") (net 1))
 (segment (start 63.5 59.944) (end 63.5 58.42) (width 1) (layer "B.Cu") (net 1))
 (segment (start 50.927 58.42) (end 52.959 60.452) (width 1) (layer "B.Cu") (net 1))
 (segment (start 52.959 60.452) (end 62.992 60.452) (width 1) (layer "B.Cu") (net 1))
 (segment (start 66.04 58.42) (end 63.5 58.42) (width 1) (layer "B.Cu") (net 1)))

